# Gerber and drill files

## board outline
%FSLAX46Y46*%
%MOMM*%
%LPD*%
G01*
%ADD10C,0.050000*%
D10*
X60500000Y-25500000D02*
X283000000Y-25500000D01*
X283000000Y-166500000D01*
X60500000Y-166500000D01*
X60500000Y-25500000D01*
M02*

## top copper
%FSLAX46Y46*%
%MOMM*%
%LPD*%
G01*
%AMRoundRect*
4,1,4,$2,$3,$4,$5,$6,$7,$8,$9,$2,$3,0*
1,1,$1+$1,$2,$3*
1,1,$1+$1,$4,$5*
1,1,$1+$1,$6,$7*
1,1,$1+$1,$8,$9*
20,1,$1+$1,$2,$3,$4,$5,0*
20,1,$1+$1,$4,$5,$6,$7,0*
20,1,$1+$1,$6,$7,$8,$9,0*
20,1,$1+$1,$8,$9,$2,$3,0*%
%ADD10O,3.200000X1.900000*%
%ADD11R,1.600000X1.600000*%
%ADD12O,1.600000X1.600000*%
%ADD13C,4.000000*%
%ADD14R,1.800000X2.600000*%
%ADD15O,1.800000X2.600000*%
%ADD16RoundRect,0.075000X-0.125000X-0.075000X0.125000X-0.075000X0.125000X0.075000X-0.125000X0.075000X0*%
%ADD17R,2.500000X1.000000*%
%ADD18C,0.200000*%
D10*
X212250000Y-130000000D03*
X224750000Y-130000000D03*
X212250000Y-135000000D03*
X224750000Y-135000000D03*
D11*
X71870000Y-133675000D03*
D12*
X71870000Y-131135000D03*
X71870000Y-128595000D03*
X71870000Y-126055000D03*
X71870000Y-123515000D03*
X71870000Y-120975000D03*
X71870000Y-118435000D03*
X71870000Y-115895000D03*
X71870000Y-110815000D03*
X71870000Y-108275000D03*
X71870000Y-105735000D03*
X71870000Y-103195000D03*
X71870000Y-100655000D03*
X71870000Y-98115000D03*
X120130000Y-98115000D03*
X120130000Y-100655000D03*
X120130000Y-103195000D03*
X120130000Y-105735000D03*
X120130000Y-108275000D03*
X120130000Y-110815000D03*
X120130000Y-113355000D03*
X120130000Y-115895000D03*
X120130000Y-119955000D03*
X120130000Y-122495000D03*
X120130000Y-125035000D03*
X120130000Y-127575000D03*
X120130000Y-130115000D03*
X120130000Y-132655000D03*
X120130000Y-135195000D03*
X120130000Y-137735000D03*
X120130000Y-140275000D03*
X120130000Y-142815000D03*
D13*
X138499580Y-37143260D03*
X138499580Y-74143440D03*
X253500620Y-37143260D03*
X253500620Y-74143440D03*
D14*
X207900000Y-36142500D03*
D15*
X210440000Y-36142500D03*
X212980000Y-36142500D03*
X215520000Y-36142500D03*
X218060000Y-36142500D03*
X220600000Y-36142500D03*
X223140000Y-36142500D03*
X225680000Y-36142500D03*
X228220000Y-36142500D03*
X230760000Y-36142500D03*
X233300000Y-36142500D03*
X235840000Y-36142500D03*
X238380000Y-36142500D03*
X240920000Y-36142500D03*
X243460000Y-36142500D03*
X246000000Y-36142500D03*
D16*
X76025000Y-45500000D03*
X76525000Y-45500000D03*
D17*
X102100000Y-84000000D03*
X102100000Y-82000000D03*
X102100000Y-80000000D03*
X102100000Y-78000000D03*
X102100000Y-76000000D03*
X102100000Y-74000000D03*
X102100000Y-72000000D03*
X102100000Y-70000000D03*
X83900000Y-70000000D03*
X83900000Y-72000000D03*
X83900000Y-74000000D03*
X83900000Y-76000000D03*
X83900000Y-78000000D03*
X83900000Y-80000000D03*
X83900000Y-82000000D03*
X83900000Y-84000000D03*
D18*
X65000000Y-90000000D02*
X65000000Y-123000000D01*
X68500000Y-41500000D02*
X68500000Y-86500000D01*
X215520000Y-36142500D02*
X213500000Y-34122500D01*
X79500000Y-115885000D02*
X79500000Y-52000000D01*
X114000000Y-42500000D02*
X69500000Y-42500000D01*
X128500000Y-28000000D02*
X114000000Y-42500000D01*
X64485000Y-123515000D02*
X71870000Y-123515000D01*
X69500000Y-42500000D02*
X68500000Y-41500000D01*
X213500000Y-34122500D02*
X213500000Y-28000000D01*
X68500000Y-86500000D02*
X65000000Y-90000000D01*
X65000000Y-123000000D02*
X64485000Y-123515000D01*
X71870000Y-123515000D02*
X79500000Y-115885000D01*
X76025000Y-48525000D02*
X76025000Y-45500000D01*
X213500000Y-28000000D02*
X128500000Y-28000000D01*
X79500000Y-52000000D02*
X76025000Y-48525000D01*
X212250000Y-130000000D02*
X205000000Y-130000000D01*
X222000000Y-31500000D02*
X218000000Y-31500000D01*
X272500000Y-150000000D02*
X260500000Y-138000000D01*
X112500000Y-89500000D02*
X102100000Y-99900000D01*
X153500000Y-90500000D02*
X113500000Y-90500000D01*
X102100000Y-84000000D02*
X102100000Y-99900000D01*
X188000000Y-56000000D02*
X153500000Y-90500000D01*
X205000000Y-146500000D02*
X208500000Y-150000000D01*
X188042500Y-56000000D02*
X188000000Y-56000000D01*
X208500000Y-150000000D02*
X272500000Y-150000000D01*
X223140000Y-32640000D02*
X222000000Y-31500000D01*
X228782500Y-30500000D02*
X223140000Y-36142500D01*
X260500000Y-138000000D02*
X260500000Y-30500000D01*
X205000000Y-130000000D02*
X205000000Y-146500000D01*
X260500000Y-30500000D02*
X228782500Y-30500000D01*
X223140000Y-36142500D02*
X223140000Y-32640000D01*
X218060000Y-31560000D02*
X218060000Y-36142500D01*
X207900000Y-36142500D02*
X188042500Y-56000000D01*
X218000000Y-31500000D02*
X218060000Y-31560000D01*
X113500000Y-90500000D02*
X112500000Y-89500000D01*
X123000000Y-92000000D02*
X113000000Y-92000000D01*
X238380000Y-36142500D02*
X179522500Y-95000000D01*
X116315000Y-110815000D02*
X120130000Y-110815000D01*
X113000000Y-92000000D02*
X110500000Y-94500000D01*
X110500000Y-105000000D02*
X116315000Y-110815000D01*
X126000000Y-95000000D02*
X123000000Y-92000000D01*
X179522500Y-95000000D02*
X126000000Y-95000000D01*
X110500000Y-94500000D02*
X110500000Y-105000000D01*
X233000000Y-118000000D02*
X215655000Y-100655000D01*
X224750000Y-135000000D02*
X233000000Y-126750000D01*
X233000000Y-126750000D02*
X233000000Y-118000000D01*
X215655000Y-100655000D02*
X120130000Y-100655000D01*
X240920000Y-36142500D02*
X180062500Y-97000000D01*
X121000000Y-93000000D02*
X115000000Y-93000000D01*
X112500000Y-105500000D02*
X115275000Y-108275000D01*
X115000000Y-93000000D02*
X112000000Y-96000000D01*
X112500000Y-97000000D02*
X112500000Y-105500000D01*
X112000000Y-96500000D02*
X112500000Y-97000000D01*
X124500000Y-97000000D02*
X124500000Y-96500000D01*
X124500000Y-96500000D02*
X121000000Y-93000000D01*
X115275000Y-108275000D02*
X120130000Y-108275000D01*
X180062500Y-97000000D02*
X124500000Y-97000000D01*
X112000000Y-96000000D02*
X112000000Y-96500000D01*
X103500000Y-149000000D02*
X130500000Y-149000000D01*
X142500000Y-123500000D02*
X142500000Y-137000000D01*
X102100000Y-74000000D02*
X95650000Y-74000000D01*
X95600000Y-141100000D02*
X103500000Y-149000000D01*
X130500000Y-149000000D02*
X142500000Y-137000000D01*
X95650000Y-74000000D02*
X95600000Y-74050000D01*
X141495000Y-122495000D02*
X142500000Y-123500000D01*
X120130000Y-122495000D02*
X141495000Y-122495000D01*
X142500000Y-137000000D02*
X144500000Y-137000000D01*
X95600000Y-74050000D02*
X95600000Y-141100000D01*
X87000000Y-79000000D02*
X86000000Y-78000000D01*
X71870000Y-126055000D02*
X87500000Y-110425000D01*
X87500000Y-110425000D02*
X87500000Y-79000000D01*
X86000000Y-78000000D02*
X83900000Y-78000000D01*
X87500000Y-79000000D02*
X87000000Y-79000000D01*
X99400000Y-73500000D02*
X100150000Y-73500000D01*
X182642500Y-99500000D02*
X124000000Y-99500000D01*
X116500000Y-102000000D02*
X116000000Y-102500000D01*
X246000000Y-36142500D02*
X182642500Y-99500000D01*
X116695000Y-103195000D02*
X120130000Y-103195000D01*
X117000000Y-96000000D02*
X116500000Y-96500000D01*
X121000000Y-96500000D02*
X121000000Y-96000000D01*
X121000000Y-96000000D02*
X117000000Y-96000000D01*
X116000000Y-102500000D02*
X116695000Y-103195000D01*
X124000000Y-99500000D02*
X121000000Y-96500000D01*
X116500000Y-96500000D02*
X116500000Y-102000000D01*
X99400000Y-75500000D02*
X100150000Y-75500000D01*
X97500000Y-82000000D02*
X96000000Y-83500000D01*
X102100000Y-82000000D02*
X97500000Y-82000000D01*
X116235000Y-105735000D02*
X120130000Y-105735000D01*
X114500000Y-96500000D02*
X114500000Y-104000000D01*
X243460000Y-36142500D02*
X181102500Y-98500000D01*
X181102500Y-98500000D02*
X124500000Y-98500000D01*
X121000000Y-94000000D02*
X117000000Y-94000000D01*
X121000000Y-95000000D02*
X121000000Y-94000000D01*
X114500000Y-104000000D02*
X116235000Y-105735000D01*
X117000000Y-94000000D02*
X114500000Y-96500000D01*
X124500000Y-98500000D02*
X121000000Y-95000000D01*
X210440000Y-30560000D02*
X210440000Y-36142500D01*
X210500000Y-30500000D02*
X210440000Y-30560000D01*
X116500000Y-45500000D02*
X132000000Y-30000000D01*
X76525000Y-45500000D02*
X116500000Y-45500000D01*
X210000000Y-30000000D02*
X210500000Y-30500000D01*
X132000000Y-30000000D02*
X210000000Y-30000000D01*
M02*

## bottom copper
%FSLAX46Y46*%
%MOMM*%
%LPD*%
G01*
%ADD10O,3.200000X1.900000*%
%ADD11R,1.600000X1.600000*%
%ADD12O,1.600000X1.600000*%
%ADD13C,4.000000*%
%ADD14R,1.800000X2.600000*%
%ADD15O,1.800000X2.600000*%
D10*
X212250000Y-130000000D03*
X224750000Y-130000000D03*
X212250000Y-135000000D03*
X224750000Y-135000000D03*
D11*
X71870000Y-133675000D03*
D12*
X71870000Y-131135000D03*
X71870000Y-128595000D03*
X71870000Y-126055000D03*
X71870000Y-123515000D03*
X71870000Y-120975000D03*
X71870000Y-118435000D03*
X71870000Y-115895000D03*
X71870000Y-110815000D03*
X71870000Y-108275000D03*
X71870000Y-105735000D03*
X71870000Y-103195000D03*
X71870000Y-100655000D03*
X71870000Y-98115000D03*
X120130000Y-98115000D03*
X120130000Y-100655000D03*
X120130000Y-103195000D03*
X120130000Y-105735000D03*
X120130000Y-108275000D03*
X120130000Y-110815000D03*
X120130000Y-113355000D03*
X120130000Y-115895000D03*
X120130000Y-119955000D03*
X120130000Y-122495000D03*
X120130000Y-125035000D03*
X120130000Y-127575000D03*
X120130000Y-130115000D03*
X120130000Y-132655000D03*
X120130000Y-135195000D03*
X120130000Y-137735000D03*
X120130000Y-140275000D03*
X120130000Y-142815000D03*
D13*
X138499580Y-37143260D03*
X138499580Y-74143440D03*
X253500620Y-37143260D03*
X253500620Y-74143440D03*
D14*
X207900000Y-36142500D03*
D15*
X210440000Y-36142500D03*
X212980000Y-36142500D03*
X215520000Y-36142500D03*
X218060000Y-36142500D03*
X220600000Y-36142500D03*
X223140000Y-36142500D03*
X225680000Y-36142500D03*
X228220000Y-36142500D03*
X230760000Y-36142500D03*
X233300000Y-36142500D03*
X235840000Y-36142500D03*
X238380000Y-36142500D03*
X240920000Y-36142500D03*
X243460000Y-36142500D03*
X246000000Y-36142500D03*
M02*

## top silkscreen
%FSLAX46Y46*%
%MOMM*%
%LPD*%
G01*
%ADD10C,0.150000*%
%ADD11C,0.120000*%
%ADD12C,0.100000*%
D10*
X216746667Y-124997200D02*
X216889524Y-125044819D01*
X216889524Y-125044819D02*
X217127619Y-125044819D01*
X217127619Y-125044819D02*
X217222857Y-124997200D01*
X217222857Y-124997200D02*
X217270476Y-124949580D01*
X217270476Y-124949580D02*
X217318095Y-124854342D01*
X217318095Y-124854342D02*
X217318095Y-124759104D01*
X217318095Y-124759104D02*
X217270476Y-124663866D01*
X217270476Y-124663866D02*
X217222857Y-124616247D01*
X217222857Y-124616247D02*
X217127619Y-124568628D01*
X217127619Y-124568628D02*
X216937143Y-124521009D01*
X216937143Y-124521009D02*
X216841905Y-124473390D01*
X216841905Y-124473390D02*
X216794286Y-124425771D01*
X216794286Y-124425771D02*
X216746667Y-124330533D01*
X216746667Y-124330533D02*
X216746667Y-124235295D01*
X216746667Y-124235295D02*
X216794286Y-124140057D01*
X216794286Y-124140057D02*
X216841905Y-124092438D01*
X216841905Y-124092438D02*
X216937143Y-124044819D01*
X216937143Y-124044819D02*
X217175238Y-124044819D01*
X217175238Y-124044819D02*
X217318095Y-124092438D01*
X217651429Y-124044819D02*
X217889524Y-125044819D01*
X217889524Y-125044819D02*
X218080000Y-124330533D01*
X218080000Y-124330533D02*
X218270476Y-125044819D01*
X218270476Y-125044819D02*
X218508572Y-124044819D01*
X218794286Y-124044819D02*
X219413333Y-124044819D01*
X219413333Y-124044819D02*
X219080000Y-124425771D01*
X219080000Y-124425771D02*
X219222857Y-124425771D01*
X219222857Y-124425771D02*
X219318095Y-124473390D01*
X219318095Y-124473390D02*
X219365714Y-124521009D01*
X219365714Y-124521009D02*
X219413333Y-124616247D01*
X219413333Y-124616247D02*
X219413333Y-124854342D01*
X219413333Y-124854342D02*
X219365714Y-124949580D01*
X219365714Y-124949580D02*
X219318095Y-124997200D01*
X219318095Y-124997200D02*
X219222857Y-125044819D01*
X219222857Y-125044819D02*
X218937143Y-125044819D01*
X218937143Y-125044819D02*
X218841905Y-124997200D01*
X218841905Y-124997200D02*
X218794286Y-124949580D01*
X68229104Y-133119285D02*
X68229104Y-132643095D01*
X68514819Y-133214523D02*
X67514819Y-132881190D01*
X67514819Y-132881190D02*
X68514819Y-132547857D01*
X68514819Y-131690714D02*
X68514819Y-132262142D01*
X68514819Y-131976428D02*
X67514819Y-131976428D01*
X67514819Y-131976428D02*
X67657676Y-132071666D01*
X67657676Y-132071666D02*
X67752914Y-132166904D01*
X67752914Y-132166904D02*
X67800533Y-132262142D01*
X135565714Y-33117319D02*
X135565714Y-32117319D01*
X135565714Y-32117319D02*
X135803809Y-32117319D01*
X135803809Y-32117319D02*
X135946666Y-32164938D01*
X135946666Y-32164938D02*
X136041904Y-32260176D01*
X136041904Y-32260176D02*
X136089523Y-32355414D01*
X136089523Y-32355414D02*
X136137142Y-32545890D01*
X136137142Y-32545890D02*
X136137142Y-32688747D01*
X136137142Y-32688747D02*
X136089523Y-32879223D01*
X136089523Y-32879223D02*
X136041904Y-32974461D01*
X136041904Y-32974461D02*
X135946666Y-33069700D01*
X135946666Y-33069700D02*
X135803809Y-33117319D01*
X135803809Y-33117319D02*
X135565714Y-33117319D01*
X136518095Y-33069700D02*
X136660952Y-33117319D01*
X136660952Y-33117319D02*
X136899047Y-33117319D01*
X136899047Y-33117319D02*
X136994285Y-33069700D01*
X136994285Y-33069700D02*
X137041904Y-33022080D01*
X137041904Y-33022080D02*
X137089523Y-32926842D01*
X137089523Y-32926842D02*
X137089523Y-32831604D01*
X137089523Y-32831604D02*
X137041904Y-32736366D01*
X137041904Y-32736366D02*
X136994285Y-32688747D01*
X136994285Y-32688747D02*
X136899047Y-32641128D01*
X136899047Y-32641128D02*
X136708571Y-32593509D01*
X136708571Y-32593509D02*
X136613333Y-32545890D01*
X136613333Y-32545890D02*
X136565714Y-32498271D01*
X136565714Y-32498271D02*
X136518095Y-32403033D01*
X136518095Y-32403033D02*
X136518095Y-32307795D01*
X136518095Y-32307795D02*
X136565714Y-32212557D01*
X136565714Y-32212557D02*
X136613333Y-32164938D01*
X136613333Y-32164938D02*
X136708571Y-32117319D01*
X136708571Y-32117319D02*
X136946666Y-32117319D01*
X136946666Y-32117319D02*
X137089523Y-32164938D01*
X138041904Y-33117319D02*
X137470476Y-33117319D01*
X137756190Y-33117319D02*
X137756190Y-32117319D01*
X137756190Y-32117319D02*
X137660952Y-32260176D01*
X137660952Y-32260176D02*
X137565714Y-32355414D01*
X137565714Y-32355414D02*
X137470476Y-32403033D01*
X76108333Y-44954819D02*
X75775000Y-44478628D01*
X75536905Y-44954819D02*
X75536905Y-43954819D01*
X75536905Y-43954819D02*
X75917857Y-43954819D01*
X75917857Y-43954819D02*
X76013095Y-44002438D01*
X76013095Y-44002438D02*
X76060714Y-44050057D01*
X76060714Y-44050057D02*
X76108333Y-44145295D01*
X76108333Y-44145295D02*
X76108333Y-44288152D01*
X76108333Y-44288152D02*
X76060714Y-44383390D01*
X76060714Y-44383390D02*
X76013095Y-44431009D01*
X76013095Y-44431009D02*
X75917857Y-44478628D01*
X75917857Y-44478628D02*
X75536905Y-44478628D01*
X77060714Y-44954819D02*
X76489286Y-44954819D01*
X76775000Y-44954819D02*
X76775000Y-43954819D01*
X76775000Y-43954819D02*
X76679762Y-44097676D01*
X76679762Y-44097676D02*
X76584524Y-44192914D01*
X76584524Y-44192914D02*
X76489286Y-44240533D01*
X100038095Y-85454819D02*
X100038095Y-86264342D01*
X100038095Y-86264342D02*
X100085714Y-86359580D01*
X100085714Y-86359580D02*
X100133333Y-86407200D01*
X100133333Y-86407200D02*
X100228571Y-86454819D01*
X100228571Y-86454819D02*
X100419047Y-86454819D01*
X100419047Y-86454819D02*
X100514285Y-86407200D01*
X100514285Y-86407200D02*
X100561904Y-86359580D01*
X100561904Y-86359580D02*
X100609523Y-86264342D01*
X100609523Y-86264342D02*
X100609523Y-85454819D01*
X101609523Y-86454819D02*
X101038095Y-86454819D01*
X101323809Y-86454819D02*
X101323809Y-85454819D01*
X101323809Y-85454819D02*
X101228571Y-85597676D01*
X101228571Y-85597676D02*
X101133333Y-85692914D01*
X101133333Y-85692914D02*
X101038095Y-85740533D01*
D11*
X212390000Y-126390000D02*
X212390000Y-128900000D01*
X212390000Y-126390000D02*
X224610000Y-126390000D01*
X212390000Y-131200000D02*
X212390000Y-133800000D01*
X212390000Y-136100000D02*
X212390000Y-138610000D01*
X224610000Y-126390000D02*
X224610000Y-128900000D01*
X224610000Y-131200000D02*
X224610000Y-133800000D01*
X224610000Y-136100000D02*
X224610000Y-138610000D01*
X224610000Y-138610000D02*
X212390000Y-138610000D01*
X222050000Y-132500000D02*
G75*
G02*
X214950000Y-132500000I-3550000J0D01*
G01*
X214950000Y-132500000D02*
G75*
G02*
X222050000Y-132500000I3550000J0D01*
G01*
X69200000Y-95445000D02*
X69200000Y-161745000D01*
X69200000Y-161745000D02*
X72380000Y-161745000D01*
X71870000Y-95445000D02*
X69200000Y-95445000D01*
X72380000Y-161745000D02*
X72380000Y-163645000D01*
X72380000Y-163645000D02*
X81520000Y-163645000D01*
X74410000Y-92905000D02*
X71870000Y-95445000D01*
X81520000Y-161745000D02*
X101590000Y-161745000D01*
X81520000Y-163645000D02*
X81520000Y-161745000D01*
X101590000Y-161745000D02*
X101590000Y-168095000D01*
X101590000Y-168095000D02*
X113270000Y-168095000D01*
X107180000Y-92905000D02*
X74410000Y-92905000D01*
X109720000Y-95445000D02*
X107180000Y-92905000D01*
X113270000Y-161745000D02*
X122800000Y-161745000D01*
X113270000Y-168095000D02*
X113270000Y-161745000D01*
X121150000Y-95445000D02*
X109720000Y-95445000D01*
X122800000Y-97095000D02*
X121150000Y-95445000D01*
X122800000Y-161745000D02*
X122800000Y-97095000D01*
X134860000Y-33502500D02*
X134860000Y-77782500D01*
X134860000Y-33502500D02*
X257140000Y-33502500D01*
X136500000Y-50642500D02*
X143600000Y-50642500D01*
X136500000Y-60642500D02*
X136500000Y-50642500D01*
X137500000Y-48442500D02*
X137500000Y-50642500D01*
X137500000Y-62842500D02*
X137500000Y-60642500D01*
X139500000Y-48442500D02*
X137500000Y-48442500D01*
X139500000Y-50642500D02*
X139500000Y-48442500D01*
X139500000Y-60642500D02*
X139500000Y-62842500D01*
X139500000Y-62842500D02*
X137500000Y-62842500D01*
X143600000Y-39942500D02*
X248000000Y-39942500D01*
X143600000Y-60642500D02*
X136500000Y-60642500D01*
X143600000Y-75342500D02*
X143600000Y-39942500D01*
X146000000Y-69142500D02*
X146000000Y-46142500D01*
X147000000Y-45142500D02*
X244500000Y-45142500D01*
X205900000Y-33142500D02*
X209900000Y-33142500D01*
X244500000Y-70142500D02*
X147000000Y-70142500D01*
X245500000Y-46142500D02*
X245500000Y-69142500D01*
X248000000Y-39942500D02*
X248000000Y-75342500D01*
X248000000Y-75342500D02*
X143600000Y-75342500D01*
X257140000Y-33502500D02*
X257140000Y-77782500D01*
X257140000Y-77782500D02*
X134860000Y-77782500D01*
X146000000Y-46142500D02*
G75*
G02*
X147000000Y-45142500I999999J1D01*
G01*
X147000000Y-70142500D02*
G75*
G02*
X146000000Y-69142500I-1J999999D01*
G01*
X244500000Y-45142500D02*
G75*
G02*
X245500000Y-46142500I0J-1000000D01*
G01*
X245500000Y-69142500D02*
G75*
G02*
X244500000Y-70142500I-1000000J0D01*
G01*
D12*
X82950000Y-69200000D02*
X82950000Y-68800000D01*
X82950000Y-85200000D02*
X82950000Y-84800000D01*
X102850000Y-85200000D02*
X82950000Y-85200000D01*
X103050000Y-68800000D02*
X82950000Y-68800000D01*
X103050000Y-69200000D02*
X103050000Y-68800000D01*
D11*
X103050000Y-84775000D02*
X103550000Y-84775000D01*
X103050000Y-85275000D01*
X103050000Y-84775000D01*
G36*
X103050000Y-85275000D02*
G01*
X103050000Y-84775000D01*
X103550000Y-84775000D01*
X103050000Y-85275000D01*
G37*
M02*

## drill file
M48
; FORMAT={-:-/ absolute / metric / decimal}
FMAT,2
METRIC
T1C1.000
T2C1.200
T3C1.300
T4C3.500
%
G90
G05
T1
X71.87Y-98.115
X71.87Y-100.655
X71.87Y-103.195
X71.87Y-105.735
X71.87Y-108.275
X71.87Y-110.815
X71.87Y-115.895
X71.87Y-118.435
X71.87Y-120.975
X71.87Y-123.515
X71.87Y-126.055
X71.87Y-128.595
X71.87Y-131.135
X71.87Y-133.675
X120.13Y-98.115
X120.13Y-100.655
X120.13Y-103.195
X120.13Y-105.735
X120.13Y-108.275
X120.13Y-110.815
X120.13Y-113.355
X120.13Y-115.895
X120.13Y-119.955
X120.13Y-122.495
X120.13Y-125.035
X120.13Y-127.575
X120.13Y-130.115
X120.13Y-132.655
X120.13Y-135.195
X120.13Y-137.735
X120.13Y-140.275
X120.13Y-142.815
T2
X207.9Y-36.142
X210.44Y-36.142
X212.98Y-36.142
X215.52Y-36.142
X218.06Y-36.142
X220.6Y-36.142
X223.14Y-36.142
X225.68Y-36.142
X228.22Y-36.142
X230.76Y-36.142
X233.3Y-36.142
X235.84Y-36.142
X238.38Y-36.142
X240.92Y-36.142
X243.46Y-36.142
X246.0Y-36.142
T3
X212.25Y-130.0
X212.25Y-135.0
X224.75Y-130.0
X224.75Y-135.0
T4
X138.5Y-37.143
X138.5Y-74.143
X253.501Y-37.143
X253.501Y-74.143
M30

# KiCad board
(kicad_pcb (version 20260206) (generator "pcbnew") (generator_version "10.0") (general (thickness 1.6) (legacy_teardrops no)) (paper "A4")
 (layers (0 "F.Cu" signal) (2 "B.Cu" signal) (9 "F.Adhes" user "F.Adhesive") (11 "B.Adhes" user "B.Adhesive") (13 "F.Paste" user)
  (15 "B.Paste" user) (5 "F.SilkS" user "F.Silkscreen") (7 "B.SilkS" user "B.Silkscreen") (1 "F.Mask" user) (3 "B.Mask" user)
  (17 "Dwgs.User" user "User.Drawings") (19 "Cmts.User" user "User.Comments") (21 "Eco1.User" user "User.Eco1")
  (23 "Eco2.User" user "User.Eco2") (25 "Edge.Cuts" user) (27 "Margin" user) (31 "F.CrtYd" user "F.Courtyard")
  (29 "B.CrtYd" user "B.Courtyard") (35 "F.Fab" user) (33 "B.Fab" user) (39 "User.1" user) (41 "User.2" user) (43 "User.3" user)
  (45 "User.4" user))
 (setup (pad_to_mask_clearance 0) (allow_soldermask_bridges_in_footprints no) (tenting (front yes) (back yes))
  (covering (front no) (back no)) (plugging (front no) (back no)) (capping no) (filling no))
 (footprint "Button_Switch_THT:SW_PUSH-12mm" (layer "F.Cu") (at 212.25 130)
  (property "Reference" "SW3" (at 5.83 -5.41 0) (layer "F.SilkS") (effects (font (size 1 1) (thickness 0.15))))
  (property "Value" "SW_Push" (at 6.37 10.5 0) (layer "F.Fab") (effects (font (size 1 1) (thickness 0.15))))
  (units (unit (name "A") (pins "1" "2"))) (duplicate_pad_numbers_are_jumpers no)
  (fp_line (start 0.14 -3.61) (end 0.14 -1.1) (stroke (width 0.12) (type default)) (layer "F.SilkS"))
  (fp_line (start 0.14 -3.61) (end 12.36 -3.61) (stroke (width 0.12) (type default)) (layer "F.SilkS"))
  (fp_line (start 0.14 1.2) (end 0.14 3.8) (stroke (width 0.12) (type default)) (layer "F.SilkS"))
  (fp_line (start 0.14 6.1) (end 0.14 8.61) (stroke (width 0.12) (type default)) (layer "F.SilkS"))
  (fp_line (start 12.36 -3.61) (end 12.36 -1.1) (stroke (width 0.12) (type default)) (layer "F.SilkS"))
  (fp_line (start 12.36 1.2) (end 12.36 3.8) (stroke (width 0.12) (type default)) (layer "F.SilkS"))
  (fp_line (start 12.36 6.1) (end 12.36 8.61) (stroke (width 0.12) (type default)) (layer "F.SilkS"))
  (fp_line (start 12.36 8.61) (end 0.14 8.61) (stroke (width 0.12) (type default)) (layer "F.SilkS"))
  (fp_circle (center 6.25 2.5) (end 9.8 2.5) (stroke (width 0.12) (type default)) (fill no) (layer "F.SilkS"))
  (pad "1" thru_hole oval (at 0 0) (size 3.2 1.9) (drill 1.3) (layers "*.Cu" "*.Mask") (remove_unused_layers no) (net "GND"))
  (pad "1" thru_hole oval (at 12.5 0) (size 3.2 1.9) (drill 1.3) (layers "*.Cu" "*.Mask") (remove_unused_layers no) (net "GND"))
  (pad "2" thru_hole oval (at 0 5) (size 3.2 1.9) (drill 1.3) (layers "*.Cu" "*.Mask") (remove_unused_layers no)
   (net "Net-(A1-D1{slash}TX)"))
  (pad "2" thru_hole oval (at 12.5 5) (size 3.2 1.9) (drill 1.3) (layers "*.Cu" "*.Mask") (remove_unused_layers no)
   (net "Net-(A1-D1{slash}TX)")))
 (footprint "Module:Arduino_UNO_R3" (layer "F.Cu") (at 71.87 133.675 90)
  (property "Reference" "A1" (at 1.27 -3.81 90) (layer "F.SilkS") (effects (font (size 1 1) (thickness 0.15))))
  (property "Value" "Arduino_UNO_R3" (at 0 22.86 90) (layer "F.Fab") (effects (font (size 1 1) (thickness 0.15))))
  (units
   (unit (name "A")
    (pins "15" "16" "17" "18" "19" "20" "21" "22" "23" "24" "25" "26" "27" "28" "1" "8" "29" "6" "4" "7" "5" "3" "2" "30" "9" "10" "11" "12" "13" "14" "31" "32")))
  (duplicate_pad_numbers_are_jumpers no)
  (fp_line (start 38.23 -2.67) (end -28.07 -2.67) (stroke (width 0.12) (type solid)) (layer "F.SilkS"))
  (fp_line (start -28.07 -2.67) (end -28.07 0.51) (stroke (width 0.12) (type solid)) (layer "F.SilkS"))
  (fp_line (start 38.23 0) (end 38.23 -2.67) (stroke (width 0.12) (type solid)) (layer "F.SilkS"))
  (fp_line (start -28.07 0.51) (end -29.97 0.51) (stroke (width 0.12) (type solid)) (layer "F.SilkS"))
  (fp_line (start -29.97 0.51) (end -29.97 9.65) (stroke (width 0.12) (type solid)) (layer "F.SilkS"))
  (fp_line (start 40.77 2.54) (end 38.23 0) (stroke (width 0.12) (type solid)) (layer "F.SilkS"))
  (fp_line (start -28.07 9.65) (end -28.07 29.72) (stroke (width 0.12) (type solid)) (layer "F.SilkS"))
  (fp_line (start -29.97 9.65) (end -28.07 9.65) (stroke (width 0.12) (type solid)) (layer "F.SilkS"))
  (fp_line (start -28.07 29.72) (end -34.42 29.72) (stroke (width 0.12) (type solid)) (layer "F.SilkS"))
  (fp_line (start -34.42 29.72) (end -34.42 41.4) (stroke (width 0.12) (type solid)) (layer "F.SilkS"))
  (fp_line (start 40.77 35.31) (end 40.77 2.54) (stroke (width 0.12) (type solid)) (layer "F.SilkS"))
  (fp_line (start 38.23 37.85) (end 40.77 35.31) (stroke (width 0.12) (type solid)) (layer "F.SilkS"))
  (fp_line (start -28.07 41.4) (end -28.07 50.93) (stroke (width 0.12) (type solid)) (layer "F.SilkS"))
  (fp_line (start -34.42 41.4) (end -28.07 41.4) (stroke (width 0.12) (type solid)) (layer "F.SilkS"))
  (fp_line (start 38.23 49.28) (end 38.23 37.85) (stroke (width 0.12) (type solid)) (layer "F.SilkS"))
  (fp_line (start 36.58 50.93) (end 38.23 49.28) (stroke (width 0.12) (type solid)) (layer "F.SilkS"))
  (fp_line (start -28.07 50.93) (end 36.58 50.93) (stroke (width 0.12) (type solid)) (layer "F.SilkS"))
  (pad "1" thru_hole rect (at 0 0 180) (size 1.6 1.6) (drill 1) (layers "*.Cu" "*.Mask") (remove_unused_layers no)
   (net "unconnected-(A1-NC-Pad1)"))
  (pad "2" thru_hole oval (at 2.54 0 180) (size 1.6 1.6) (drill 1) (layers "*.Cu" "*.Mask") (remove_unused_layers no)
   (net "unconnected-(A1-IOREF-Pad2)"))
  (pad "3" thru_hole oval (at 5.08 0 180) (size 1.6 1.6) (drill 1) (layers "*.Cu" "*.Mask") (remove_unused_layers no)
   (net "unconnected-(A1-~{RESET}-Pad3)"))
  (pad "4" thru_hole oval (at 7.62 0 180) (size 1.6 1.6) (drill 1) (layers "*.Cu" "*.Mask") (remove_unused_layers no) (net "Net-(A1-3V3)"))
  (pad "5" thru_hole oval (at 10.16 0 180) (size 1.6 1.6) (drill 1) (layers "*.Cu" "*.Mask") (remove_unused_layers no) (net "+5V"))
  (pad "6" thru_hole oval (at 12.7 0 180) (size 1.6 1.6) (drill 1) (layers "*.Cu" "*.Mask") (remove_unused_layers no)
   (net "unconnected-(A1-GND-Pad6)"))
  (pad "7" thru_hole oval (at 15.24 0 180) (size 1.6 1.6) (drill 1) (layers "*.Cu" "*.Mask") (remove_unused_layers no)
   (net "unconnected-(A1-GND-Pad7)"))
  (pad "8" thru_hole oval (at 17.78 0 180) (size 1.6 1.6) (drill 1) (layers "*.Cu" "*.Mask") (remove_unused_layers no)
   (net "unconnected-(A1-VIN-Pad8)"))
  (pad "9" thru_hole oval (at 22.86 0 180) (size 1.6 1.6) (drill 1) (layers "*.Cu" "*.Mask") (remove_unused_layers no)
   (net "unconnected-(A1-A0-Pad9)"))
  (pad "10" thru_hole oval (at 25.4 0 180) (size 1.6 1.6) (drill 1) (layers "*.Cu" "*.Mask") (remove_unused_layers no)
   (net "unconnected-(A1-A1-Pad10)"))
  (pad "11" thru_hole oval (at 27.94 0 180) (size 1.6 1.6) (drill 1) (layers "*.Cu" "*.Mask") (remove_unused_layers no)
   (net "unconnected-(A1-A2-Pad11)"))
  (pad "12" thru_hole oval (at 30.48 0 180) (size 1.6 1.6) (drill 1) (layers "*.Cu" "*.Mask") (remove_unused_layers no)
   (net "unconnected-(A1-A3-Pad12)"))
  (pad "13" thru_hole oval (at 33.02 0 180) (size 1.6 1.6) (drill 1) (layers "*.Cu" "*.Mask") (remove_unused_layers no)
   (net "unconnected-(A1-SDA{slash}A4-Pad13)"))
  (pad "14" thru_hole oval (at 35.56 0 180) (size 1.6 1.6) (drill 1) (layers "*.Cu" "*.Mask") (remove_unused_layers no)
   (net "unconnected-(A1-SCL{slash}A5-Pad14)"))
  (pad "15" thru_hole oval (at 35.56 48.26 180) (size 1.6 1.6) (drill 1) (layers "*.Cu" "*.Mask") (remove_unused_layers no)
   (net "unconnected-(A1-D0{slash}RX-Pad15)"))
  (pad "16" thru_hole oval (at 33.02 48.26 180) (size 1.6 1.6) (drill 1) (layers "*.Cu" "*.Mask") (remove_unused_layers no)
   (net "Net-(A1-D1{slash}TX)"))
  (pad "17" thru_hole oval (at 30.48 48.26 180) (size 1.6 1.6) (drill 1) (layers "*.Cu" "*.Mask") (remove_unused_layers no)
   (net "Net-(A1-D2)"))
  (pad "18" thru_hole oval (at 27.94 48.26 180) (size 1.6 1.6) (drill 1) (layers "*.Cu" "*.Mask") (remove_unused_layers no)
   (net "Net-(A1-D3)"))
  (pad "19" thru_hole oval (at 25.4 48.26 180) (size 1.6 1.6) (drill 1) (layers "*.Cu" "*.Mask") (remove_unused_layers no)
   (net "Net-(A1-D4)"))
  (pad "20" thru_hole oval (at 22.86 48.26 180) (size 1.6 1.6) (drill 1) (layers "*.Cu" "*.Mask") (remove_unused_layers no)
   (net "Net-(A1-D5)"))
  (pad "21" thru_hole oval (at 20.32 48.26 180) (size 1.6 1.6) (drill 1) (layers "*.Cu" "*.Mask") (remove_unused_layers no)
   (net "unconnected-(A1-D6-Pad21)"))
  (pad "22" thru_hole oval (at 17.78 48.26 180) (size 1.6 1.6) (drill 1) (layers "*.Cu" "*.Mask") (remove_unused_layers no)
   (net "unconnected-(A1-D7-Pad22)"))
  (pad "23" thru_hole oval (at 13.72 48.26 180) (size 1.6 1.6) (drill 1) (layers "*.Cu" "*.Mask") (remove_unused_layers no)
   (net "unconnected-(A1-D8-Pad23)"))
  (pad "24" thru_hole oval (at 11.18 48.26 180) (size 1.6 1.6) (drill 1) (layers "*.Cu" "*.Mask") (remove_unused_layers no)
   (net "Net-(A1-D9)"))
  (pad "25" thru_hole oval (at 8.64 48.26 180) (size 1.6 1.6) (drill 1) (layers "*.Cu" "*.Mask") (remove_unused_layers no)
   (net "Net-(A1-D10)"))
  (pad "26" thru_hole oval (at 6.1 48.26 180) (size 1.6 1.6) (drill 1) (layers "*.Cu" "*.Mask") (remove_unused_layers no)
   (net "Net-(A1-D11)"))
  (pad "27" thru_hole oval (at 3.56 48.26 180) (size 1.6 1.6) (drill 1) (layers "*.Cu" "*.Mask") (remove_unused_layers no)
   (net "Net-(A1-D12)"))
  (pad "28" thru_hole oval (at 1.02 48.26 180) (size 1.6 1.6) (drill 1) (layers "*.Cu" "*.Mask") (remove_unused_layers no)
   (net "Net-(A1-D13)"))
  (pad "29" thru_hole oval (at -1.52 48.26 180) (size 1.6 1.6) (drill 1) (layers "*.Cu" "*.Mask") (remove_unused_layers no) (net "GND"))
  (pad "30" thru_hole oval (at -4.06 48.26 180) (size 1.6 1.6) (drill 1) (layers "*.Cu" "*.Mask") (remove_unused_layers no)
   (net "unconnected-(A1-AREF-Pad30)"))
  (pad "31" thru_hole oval (at -6.6 48.26 180) (size 1.6 1.6) (drill 1) (layers "*.Cu" "*.Mask") (remove_unused_layers no)
   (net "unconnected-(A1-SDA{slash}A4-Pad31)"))
  (pad "32" thru_hole oval (at -9.14 48.26 180) (size 1.6 1.6) (drill 1) (layers "*.Cu" "*.Mask") (remove_unused_layers no)
   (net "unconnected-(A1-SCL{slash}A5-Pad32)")))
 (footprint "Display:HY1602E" (layer "F.Cu") (at 207.9 36.1425)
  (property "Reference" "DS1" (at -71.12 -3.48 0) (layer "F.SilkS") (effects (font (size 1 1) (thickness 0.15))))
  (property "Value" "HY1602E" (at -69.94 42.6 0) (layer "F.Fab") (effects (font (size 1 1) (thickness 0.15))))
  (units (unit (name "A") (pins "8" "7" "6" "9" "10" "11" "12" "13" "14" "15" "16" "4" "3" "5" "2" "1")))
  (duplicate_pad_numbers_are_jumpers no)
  (fp_line (start -73.04 -2.64) (end -73.04 41.64) (stroke (width 0.12) (type solid)) (layer "F.SilkS"))
  (fp_line (start -73.04 -2.64) (end 49.24 -2.64) (stroke (width 0.12) (type solid)) (layer "F.SilkS"))
  (fp_line (start -71.4 14.5) (end -64.3 14.5) (stroke (width 0.12) (type solid)) (layer "F.SilkS"))
  (fp_line (start -71.4 24.5) (end -71.4 14.5) (stroke (width 0.12) (type solid)) (layer "F.SilkS"))
  (fp_line (start -70.4 12.3) (end -70.4 14.5) (stroke (width 0.12) (type solid)) (layer "F.SilkS"))
  (fp_line (start -70.4 26.7) (end -70.4 24.5) (stroke (width 0.12) (type solid)) (layer "F.SilkS"))
  (fp_line (start -68.4 12.3) (end -70.4 12.3) (stroke (width 0.12) (type solid)) (layer "F.SilkS"))
  (fp_line (start -68.4 14.5) (end -68.4 12.3) (stroke (width 0.12) (type solid)) (layer "F.SilkS"))
  (fp_line (start -68.4 24.5) (end -68.4 26.7) (stroke (width 0.12) (type solid)) (layer "F.SilkS"))
  (fp_line (start -68.4 26.7) (end -70.4 26.7) (stroke (width 0.12) (type solid)) (layer "F.SilkS"))
  (fp_line (start -64.3 3.8) (end 40.1 3.8) (stroke (width 0.12) (type solid)) (layer "F.SilkS"))
  (fp_line (start -64.3 24.5) (end -71.4 24.5) (stroke (width 0.12) (type solid)) (layer "F.SilkS"))
  (fp_line (start -64.3 39.2) (end -64.3 3.8) (stroke (width 0.12) (type solid)) (layer "F.SilkS"))
  (fp_line (start -61.9 33) (end -61.9 10) (stroke (width 0.12) (type solid)) (layer "F.SilkS"))
  (fp_line (start -60.9 9) (end 36.6 9) (stroke (width 0.12) (type solid)) (layer "F.SilkS"))
  (fp_line (start -2 -3) (end 2 -3) (stroke (width 0.12) (type solid)) (layer "F.SilkS"))
  (fp_line (start 36.6 34) (end -60.9 34) (stroke (width 0.12) (type solid)) (layer "F.SilkS"))
  (fp_line (start 37.6 10) (end 37.6 33) (stroke (width 0.12) (type solid)) (layer "F.SilkS"))
  (fp_line (start 40.1 3.8) (end 40.1 39.2) (stroke (width 0.12) (type solid)) (layer "F.SilkS"))
  (fp_line (start 40.1 39.2) (end -64.3 39.2) (stroke (width 0.12) (type solid)) (layer "F.SilkS"))
  (fp_line (start 49.24 -2.64) (end 49.24 41.64) (stroke (width 0.12) (type solid)) (layer "F.SilkS"))
  (fp_line (start 49.24 41.64) (end -73.04 41.64) (stroke (width 0.12) (type solid)) (layer "F.SilkS"))
  (fp_arc (start -61.9 10) (mid -61.607107 9.292893) (end -60.9 9) (stroke (width 0.12) (type solid)) (layer "F.SilkS"))
  (fp_arc (start -60.9 34) (mid -61.607107 33.707107) (end -61.9 33) (stroke (width 0.12) (type solid)) (layer "F.SilkS"))
  (fp_arc (start 36.6 9) (mid 37.307107 9.292893) (end 37.6 10) (stroke (width 0.12) (type solid)) (layer "F.SilkS"))
  (fp_arc (start 37.6 33) (mid 37.307107 33.707107) (end 36.6 34) (stroke (width 0.12) (type solid)) (layer "F.SilkS"))
  (pad "" thru_hole circle (at -69.40042 1.00076 180) (size 4 4) (drill 3.5) (layers "*.Cu" "*.Mask") (remove_unused_layers no))
  (pad "" thru_hole circle (at -69.40042 38.00094 180) (size 4 4) (drill 3.5) (layers "*.Cu" "*.Mask") (remove_unused_layers no))
  (pad "" thru_hole circle (at 45.60062 1.00076 180) (size 4 4) (drill 3.5) (layers "*.Cu" "*.Mask") (remove_unused_layers no))
  (pad "" thru_hole circle (at 45.60062 38.00094 180) (size 4 4) (drill 3.5) (layers "*.Cu" "*.Mask") (remove_unused_layers no))
  (pad "1" thru_hole rect (at 0 0 180) (size 1.8 2.6) (drill 1.2) (layers "*.Cu" "*.Mask") (remove_unused_layers no) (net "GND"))
  (pad "2" thru_hole oval (at 2.54 0 180) (size 1.8 2.6) (drill 1.2) (layers "*.Cu" "*.Mask") (remove_unused_layers no)
   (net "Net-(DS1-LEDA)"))
  (pad "3" thru_hole oval (at 5.08 0 180) (size 1.8 2.6) (drill 1.2) (layers "*.Cu" "*.Mask") (remove_unused_layers no) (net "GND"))
  (pad "4" thru_hole oval (at 7.62 0 180) (size 1.8 2.6) (drill 1.2) (layers "*.Cu" "*.Mask") (remove_unused_layers no) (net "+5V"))
  (pad "5" thru_hole oval (at 10.16 0 180) (size 1.8 2.6) (drill 1.2) (layers "*.Cu" "*.Mask") (remove_unused_layers no) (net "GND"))
  (pad "6" thru_hole oval (at 12.7 0 180) (size 1.8 2.6) (drill 1.2) (layers "*.Cu" "*.Mask") (remove_unused_layers no)
   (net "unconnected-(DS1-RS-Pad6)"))
  (pad "7" thru_hole oval (at 15.24 0 180) (size 1.8 2.6) (drill 1.2) (layers "*.Cu" "*.Mask") (remove_unused_layers no) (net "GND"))
  (pad "8" thru_hole oval (at 17.78 0 180) (size 1.8 2.6) (drill 1.2) (layers "*.Cu" "*.Mask") (remove_unused_layers no)
   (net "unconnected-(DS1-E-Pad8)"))
  (pad "9" thru_hole oval (at 20.32 0 180) (size 1.8 2.6) (drill 1.2) (layers "*.Cu" "*.Mask") (remove_unused_layers no)
   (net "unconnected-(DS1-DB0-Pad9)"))
  (pad "10" thru_hole oval (at 22.86 0 180) (size 1.8 2.6) (drill 1.2) (layers "*.Cu" "*.Mask") (remove_unused_layers no)
   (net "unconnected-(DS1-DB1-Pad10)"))
  (pad "11" thru_hole oval (at 25.4 0 180) (size 1.8 2.6) (drill 1.2) (layers "*.Cu" "*.Mask") (remove_unused_layers no)
   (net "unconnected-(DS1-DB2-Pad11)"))
  (pad "12" thru_hole oval (at 27.94 0 180) (size 1.8 2.6) (drill 1.2) (layers "*.Cu" "*.Mask") (remove_unused_layers no)
   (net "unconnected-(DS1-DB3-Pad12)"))
  (pad "13" thru_hole oval (at 30.48 0 180) (size 1.8 2.6) (drill 1.2) (layers "*.Cu" "*.Mask") (remove_unused_layers no)
   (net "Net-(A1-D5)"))
  (pad "14" thru_hole oval (at 33.02 0 180) (size 1.8 2.6) (drill 1.2) (layers "*.Cu" "*.Mask") (remove_unused_layers no)
   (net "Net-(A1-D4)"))
  (pad "15" thru_hole oval (at 35.56 0 180) (size 1.8 2.6) (drill 1.2) (layers "*.Cu" "*.Mask") (remove_unused_layers no)
   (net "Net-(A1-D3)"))
  (pad "16" thru_hole oval (at 38.1 0 180) (size 1.8 2.6) (drill 1.2) (layers "*.Cu" "*.Mask") (remove_unused_layers no) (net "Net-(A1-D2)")))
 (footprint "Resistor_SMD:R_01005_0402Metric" (layer "F.Cu") (at 76.275 45.5)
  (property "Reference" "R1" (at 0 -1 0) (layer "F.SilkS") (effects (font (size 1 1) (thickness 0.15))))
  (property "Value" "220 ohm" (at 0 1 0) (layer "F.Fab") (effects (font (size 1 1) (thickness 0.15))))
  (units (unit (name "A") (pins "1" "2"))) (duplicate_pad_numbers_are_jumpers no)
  (pad "" smd roundrect (at -0.275 0) (size 0.27 0.27) (layers "F.Paste") (roundrect_rratio 0.25))
  (pad "" smd roundrect (at 0.275 0) (size 0.27 0.27) (layers "F.Paste") (roundrect_rratio 0.25))
  (pad "1" smd roundrect (at -0.25 0) (size 0.4 0.3) (layers "F.Cu" "F.Mask") (roundrect_rratio 0.25) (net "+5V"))
  (pad "2" smd roundrect (at 0.25 0) (size 0.4 0.3) (layers "F.Cu" "F.Mask") (roundrect_rratio 0.25) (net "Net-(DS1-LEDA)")))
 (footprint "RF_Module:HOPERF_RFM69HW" (layer "F.Cu") (at 93 77 180)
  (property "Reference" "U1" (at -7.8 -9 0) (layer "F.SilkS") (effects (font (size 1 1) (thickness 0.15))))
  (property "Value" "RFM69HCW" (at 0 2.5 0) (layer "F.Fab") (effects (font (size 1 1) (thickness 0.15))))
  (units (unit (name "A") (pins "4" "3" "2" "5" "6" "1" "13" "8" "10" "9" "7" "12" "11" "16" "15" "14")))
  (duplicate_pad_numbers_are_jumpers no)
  (fp_line (start 10.05 7.8) (end 10.05 8.2) (stroke (width 0.1) (type solid)) (layer "F.SilkS"))
  (fp_line (start 10.05 -8.2) (end 10.05 -7.8) (stroke (width 0.1) (type solid)) (layer "F.SilkS"))
  (fp_line (start -9.85 -8.2) (end 10.05 -8.2) (stroke (width 0.1) (type solid)) (layer "F.SilkS"))
  (fp_line (start -10.05 8.2) (end 10.05 8.2) (stroke (width 0.1) (type solid)) (layer "F.SilkS"))
  (fp_line (start -10.05 7.8) (end -10.05 8.2) (stroke (width 0.1) (type solid)) (layer "F.SilkS"))
  (fp_poly
   (pts (xy -10.05 -7.775) (xy -10.55 -7.775) (xy -10.05 -8.275) (xy -10.05 -7.775)) (stroke (width 0.12) (type solid)) (fill yes)
   (layer "F.SilkS"))
  (pad "1" smd rect (at -9.1 -7 180) (size 2.5 1) (layers "F.Cu" "F.Mask" "F.Paste") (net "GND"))
  (pad "2" smd rect (at -9.1 -5 180) (size 2.5 1) (layers "F.Cu" "F.Mask" "F.Paste") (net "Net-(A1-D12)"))
  (pad "3" smd rect (at -9.1 -3 180) (size 2.5 1) (layers "F.Cu" "F.Mask" "F.Paste") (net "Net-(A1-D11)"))
  (pad "4" smd rect (at -9.1 -1 180) (size 2.5 1) (layers "F.Cu" "F.Mask" "F.Paste") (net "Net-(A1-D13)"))
  (pad "5" smd rect (at -9.1 1 180) (size 2.5 1) (layers "F.Cu" "F.Mask" "F.Paste") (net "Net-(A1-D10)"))
  (pad "6" smd rect (at -9.1 3 180) (size 2.5 1) (layers "F.Cu" "F.Mask" "F.Paste") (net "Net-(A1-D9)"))
  (pad "7" smd rect (at -9.1 5 180) (size 2.5 1) (layers "F.Cu" "F.Mask" "F.Paste") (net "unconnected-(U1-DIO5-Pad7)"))
  (pad "8" smd rect (at -9.1 7 180) (size 2.5 1) (layers "F.Cu" "F.Mask" "F.Paste") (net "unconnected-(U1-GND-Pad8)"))
  (pad "9" smd rect (at 9.1 7 180) (size 2.5 1) (layers "F.Cu" "F.Mask" "F.Paste") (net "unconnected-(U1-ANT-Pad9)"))
  (pad "10" smd rect (at 9.1 5 180) (size 2.5 1) (layers "F.Cu" "F.Mask" "F.Paste") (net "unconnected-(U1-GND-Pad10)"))
  (pad "11" smd rect (at 9.1 3 180) (size 2.5 1) (layers "F.Cu" "F.Mask" "F.Paste") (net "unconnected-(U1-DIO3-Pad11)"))
  (pad "12" smd rect (at 9.1 1 180) (size 2.5 1) (layers "F.Cu" "F.Mask" "F.Paste") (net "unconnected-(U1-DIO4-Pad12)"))
  (pad "13" smd rect (at 9.1 -1 180) (size 2.5 1) (layers "F.Cu" "F.Mask" "F.Paste") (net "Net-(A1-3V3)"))
  (pad "14" smd rect (at 9.1 -3 180) (size 2.5 1) (layers "F.Cu" "F.Mask" "F.Paste") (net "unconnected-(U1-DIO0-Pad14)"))
  (pad "15" smd rect (at 9.1 -5 180) (size 2.5 1) (layers "F.Cu" "F.Mask" "F.Paste") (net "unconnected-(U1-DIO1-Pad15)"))
  (pad "16" smd rect (at 9.1 -7 180) (size 2.5 1) (layers "F.Cu" "F.Mask" "F.Paste") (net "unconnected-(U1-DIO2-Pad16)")))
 (gr_rect (start 60.5 25.5) (end 283 166.5) (stroke (width 0.05) (type default)) (fill no) (layer "Edge.Cuts"))
 (segment (start 65 90) (end 65 123) (width 0.2) (layer "F.Cu") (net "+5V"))
 (segment (start 68.5 41.5) (end 68.5 86.5) (width 0.2) (layer "F.Cu") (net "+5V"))
 (segment (start 215.52 36.1425) (end 213.5 34.1225) (width 0.2) (layer "F.Cu") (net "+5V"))
 (segment (start 79.5 115.885) (end 79.5 52) (width 0.2) (layer "F.Cu") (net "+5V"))
 (segment (start 114 42.5) (end 69.5 42.5) (width 0.2) (layer "F.Cu") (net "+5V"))
 (segment (start 128.5 28) (end 114 42.5) (width 0.2) (layer "F.Cu") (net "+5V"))
 (segment (start 64.485 123.515) (end 71.87 123.515) (width 0.2) (layer "F.Cu") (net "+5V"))
 (segment (start 69.5 42.5) (end 68.5 41.5) (width 0.2) (layer "F.Cu") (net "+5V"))
 (segment (start 213.5 34.1225) (end 213.5 28) (width 0.2) (layer "F.Cu") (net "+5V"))
 (segment (start 68.5 86.5) (end 65 90) (width 0.2) (layer "F.Cu") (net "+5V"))
 (segment (start 65 123) (end 64.485 123.515) (width 0.2) (layer "F.Cu") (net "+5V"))
 (segment (start 71.87 123.515) (end 79.5 115.885) (width 0.2) (layer "F.Cu") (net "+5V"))
 (segment (start 76.025 48.525) (end 76.025 45.5) (width 0.2) (layer "F.Cu") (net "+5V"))
 (segment (start 213.5 28) (end 128.5 28) (width 0.2) (layer "F.Cu") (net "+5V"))
 (segment (start 79.5 52) (end 76.025 48.525) (width 0.2) (layer "F.Cu") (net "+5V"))
 (segment (start 212.25 130) (end 205 130) (width 0.2) (layer "F.Cu") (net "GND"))
 (segment (start 222 31.5) (end 218 31.5) (width 0.2) (layer "F.Cu") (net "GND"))
 (segment (start 272.5 150) (end 260.5 138) (width 0.2) (layer "F.Cu") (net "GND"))
 (segment (start 112.5 89.5) (end 102.1 99.9) (width 0.2) (layer "F.Cu") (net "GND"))
 (segment (start 153.5 90.5) (end 113.5 90.5) (width 0.2) (layer "F.Cu") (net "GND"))
 (segment (start 102.1 84) (end 102.1 99.9) (width 0.2) (layer "F.Cu") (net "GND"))
 (segment (start 188 56) (end 153.5 90.5) (width 0.2) (layer "F.Cu") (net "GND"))
 (segment (start 205 146.5) (end 208.5 150) (width 0.2) (layer "F.Cu") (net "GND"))
 (segment (start 188.0425 56) (end 188 56) (width 0.2) (layer "F.Cu") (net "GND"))
 (segment (start 208.5 150) (end 272.5 150) (width 0.2) (layer "F.Cu") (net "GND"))
 (segment (start 223.14 32.64) (end 222 31.5) (width 0.2) (layer "F.Cu") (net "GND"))
 (segment (start 228.7825 30.5) (end 223.14 36.1425) (width 0.2) (layer "F.Cu") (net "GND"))
 (segment (start 260.5 138) (end 260.5 30.5) (width 0.2) (layer "F.Cu") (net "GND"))
 (segment (start 205 130) (end 205 146.5) (width 0.2) (layer "F.Cu") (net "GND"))
 (segment (start 260.5 30.5) (end 228.7825 30.5) (width 0.2) (layer "F.Cu") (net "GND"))
 (segment (start 223.14 36.1425) (end 223.14 32.64) (width 0.2) (layer "F.Cu") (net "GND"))
 (segment (start 218.06 31.56) (end 218.06 36.1425) (width 0.2) (layer "F.Cu") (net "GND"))
 (segment (start 207.9 36.1425) (end 188.0425 56) (width 0.2) (layer "F.Cu") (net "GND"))
 (segment (start 218 31.5) (end 218.06 31.56) (width 0.2) (layer "F.Cu") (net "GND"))
 (segment (start 113.5 90.5) (end 112.5 89.5) (width 0.2) (layer "F.Cu") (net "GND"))
 (segment (start 123 92) (end 113 92) (width 0.2) (layer "F.Cu") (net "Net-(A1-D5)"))
 (segment (start 238.38 36.1425) (end 179.5225 95) (width 0.2) (layer "F.Cu") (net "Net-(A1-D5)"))
 (segment (start 116.315 110.815) (end 120.13 110.815) (width 0.2) (layer "F.Cu") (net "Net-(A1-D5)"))
 (segment (start 113 92) (end 110.5 94.5) (width 0.2) (layer "F.Cu") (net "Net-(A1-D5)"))
 (segment (start 110.5 105) (end 116.315 110.815) (width 0.2) (layer "F.Cu") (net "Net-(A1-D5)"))
 (segment (start 126 95) (end 123 92) (width 0.2) (layer "F.Cu") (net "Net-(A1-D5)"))
 (segment (start 179.5225 95) (end 126 95) (width 0.2) (layer "F.Cu") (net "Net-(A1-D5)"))
 (segment (start 110.5 94.5) (end 110.5 105) (width 0.2) (layer "F.Cu") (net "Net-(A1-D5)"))
 (segment (start 233 118) (end 215.655 100.655) (width 0.2) (layer "F.Cu") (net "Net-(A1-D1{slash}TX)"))
 (segment (start 224.75 135) (end 233 126.75) (width 0.2) (layer "F.Cu") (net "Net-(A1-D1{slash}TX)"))
 (segment (start 233 126.75) (end 233 118) (width 0.2) (layer "F.Cu") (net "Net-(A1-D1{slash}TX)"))
 (segment (start 215.655 100.655) (end 120.13 100.655) (width 0.2) (layer "F.Cu") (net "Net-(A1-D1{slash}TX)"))
 (segment (start 240.92 36.1425) (end 180.0625 97) (width 0.2) (layer "F.Cu") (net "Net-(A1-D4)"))
 (segment (start 121 93) (end 115 93) (width 0.2) (layer "F.Cu") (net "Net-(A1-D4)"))
 (segment (start 112.5 105.5) (end 115.275 108.275) (width 0.2) (layer "F.Cu") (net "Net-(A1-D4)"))
 (segment (start 115 93) (end 112 96) (width 0.2) (layer "F.Cu") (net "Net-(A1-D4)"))
 (segment (start 112.5 97) (end 112.5 105.5) (width 0.2) (layer "F.Cu") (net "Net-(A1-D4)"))
 (segment (start 112 96.5) (end 112.5 97) (width 0.2) (layer "F.Cu") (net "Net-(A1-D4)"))
 (segment (start 124.5 97) (end 124.5 96.5) (width 0.2) (layer "F.Cu") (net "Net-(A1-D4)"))
 (segment (start 124.5 96.5) (end 121 93) (width 0.2) (layer "F.Cu") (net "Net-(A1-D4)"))
 (segment (start 115.275 108.275) (end 120.13 108.275) (width 0.2) (layer "F.Cu") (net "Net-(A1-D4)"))
 (segment (start 180.0625 97) (end 124.5 97) (width 0.2) (layer "F.Cu") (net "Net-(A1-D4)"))
 (segment (start 112 96) (end 112 96.5) (width 0.2) (layer "F.Cu") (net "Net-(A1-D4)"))
 (segment (start 103.5 149) (end 130.5 149) (width 0.2) (layer "F.Cu") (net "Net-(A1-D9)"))
 (segment (start 142.5 123.5) (end 142.5 137) (width 0.2) (layer "F.Cu") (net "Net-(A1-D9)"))
 (segment (start 102.1 74) (end 95.65 74) (width 0.2) (layer "F.Cu") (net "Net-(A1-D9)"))
 (segment (start 95.6 141.1) (end 103.5 149) (width 0.2) (layer "F.Cu") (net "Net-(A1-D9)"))
 (segment (start 130.5 149) (end 142.5 137) (width 0.2) (layer "F.Cu") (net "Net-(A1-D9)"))
 (segment (start 95.65 74) (end 95.6 74.05) (width 0.2) (layer "F.Cu") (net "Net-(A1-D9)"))
 (segment (start 141.495 122.495) (end 142.5 123.5) (width 0.2) (layer "F.Cu") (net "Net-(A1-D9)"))
 (segment (start 120.13 122.495) (end 141.495 122.495) (width 0.2) (layer "F.Cu") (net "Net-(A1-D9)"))
 (segment (start 142.5 137) (end 144.5 137) (width 0.2) (layer "F.Cu") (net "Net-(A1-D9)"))
 (segment (start 95.6 74.05) (end 95.6 141.1) (width 0.2) (layer "F.Cu") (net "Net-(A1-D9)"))
 (segment (start 87 79) (end 86 78) (width 0.2) (layer "F.Cu") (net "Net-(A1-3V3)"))
 (segment (start 71.87 126.055) (end 87.5 110.425) (width 0.2) (layer "F.Cu") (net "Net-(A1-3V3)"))
 (segment (start 87.5 110.425) (end 87.5 79) (width 0.2) (layer "F.Cu") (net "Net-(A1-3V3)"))
 (segment (start 86 78) (end 83.9 78) (width 0.2) (layer "F.Cu") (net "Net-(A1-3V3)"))
 (segment (start 87.5 79) (end 87 79) (width 0.2) (layer "F.Cu") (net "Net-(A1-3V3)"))
 (segment (start 99.4 73.5) (end 100.15 73.5) (width 0.2) (layer "F.Cu") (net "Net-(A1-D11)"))
 (segment (start 182.6425 99.5) (end 124 99.5) (width 0.2) (layer "F.Cu") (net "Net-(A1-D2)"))
 (segment (start 116.5 102) (end 116 102.5) (width 0.2) (layer "F.Cu") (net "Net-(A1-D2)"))
 (segment (start 246 36.1425) (end 182.6425 99.5) (width 0.2) (layer "F.Cu") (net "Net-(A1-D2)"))
 (segment (start 116.695 103.195) (end 120.13 103.195) (width 0.2) (layer "F.Cu") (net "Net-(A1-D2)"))
 (segment (start 117 96) (end 116.5 96.5) (width 0.2) (layer "F.Cu") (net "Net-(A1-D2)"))
 (segment (start 121 96.5) (end 121 96) (width 0.2) (layer "F.Cu") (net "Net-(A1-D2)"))
 (segment (start 121 96) (end 117 96) (width 0.2) (layer "F.Cu") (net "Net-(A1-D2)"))
 (segment (start 116 102.5) (end 116.695 103.195) (width 0.2) (layer "F.Cu") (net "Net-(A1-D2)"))
 (segment (start 124 99.5) (end 121 96.5) (width 0.2) (layer "F.Cu") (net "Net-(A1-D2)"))
 (segment (start 116.5 96.5) (end 116.5 102) (width 0.2) (layer "F.Cu") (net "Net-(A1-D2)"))
 (segment (start 99.4 75.5) (end 100.15 75.5) (width 0.2) (layer "F.Cu") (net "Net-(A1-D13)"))
 (segment (start 97.5 82) (end 96 83.5) (width 0.2) (layer "F.Cu") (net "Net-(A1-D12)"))
 (segment (start 102.1 82) (end 97.5 82) (width 0.2) (layer "F.Cu") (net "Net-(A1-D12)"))
 (segment (start 116.235 105.735) (end 120.13 105.735) (width 0.2) (layer "F.Cu") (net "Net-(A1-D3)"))
 (segment (start 114.5 96.5) (end 114.5 104) (width 0.2) (layer "F.Cu") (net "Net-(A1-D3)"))
 (segment (start 243.46 36.1425) (end 181.1025 98.5) (width 0.2) (layer "F.Cu") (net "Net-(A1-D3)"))
 (segment (start 181.1025 98.5) (end 124.5 98.5) (width 0.2) (layer "F.Cu") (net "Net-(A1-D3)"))
 (segment (start 121 94) (end 117 94) (width 0.2) (layer "F.Cu") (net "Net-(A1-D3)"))
 (segment (start 121 95) (end 121 94) (width 0.2) (layer "F.Cu") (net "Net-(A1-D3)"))
 (segment (start 114.5 104) (end 116.235 105.735) (width 0.2) (layer "F.Cu") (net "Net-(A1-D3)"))
 (segment (start 117 94) (end 114.5 96.5) (width 0.2) (layer "F.Cu") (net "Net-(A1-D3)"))
 (segment (start 124.5 98.5) (end 121 95) (width 0.2) (layer "F.Cu") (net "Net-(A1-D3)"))
 (segment (start 210.44 30.56) (end 210.44 36.1425) (width 0.2) (layer "F.Cu") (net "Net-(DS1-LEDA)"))
 (segment (start 210.5 30.5) (end 210.44 30.56) (width 0.2) (layer "F.Cu") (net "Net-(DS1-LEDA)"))
 (segment (start 116.5 45.5) (end 132 30) (width 0.2) (layer "F.Cu") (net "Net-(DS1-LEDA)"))
 (segment (start 76.525 45.5) (end 116.5 45.5) (width 0.2) (layer "F.Cu") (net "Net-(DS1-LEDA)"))
 (segment (start 210 30) (end 210.5 30.5) (width 0.2) (layer "F.Cu") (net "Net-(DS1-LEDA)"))
 (segment (start 132 30) (end 210 30) (width 0.2) (layer "F.Cu") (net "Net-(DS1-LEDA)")))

